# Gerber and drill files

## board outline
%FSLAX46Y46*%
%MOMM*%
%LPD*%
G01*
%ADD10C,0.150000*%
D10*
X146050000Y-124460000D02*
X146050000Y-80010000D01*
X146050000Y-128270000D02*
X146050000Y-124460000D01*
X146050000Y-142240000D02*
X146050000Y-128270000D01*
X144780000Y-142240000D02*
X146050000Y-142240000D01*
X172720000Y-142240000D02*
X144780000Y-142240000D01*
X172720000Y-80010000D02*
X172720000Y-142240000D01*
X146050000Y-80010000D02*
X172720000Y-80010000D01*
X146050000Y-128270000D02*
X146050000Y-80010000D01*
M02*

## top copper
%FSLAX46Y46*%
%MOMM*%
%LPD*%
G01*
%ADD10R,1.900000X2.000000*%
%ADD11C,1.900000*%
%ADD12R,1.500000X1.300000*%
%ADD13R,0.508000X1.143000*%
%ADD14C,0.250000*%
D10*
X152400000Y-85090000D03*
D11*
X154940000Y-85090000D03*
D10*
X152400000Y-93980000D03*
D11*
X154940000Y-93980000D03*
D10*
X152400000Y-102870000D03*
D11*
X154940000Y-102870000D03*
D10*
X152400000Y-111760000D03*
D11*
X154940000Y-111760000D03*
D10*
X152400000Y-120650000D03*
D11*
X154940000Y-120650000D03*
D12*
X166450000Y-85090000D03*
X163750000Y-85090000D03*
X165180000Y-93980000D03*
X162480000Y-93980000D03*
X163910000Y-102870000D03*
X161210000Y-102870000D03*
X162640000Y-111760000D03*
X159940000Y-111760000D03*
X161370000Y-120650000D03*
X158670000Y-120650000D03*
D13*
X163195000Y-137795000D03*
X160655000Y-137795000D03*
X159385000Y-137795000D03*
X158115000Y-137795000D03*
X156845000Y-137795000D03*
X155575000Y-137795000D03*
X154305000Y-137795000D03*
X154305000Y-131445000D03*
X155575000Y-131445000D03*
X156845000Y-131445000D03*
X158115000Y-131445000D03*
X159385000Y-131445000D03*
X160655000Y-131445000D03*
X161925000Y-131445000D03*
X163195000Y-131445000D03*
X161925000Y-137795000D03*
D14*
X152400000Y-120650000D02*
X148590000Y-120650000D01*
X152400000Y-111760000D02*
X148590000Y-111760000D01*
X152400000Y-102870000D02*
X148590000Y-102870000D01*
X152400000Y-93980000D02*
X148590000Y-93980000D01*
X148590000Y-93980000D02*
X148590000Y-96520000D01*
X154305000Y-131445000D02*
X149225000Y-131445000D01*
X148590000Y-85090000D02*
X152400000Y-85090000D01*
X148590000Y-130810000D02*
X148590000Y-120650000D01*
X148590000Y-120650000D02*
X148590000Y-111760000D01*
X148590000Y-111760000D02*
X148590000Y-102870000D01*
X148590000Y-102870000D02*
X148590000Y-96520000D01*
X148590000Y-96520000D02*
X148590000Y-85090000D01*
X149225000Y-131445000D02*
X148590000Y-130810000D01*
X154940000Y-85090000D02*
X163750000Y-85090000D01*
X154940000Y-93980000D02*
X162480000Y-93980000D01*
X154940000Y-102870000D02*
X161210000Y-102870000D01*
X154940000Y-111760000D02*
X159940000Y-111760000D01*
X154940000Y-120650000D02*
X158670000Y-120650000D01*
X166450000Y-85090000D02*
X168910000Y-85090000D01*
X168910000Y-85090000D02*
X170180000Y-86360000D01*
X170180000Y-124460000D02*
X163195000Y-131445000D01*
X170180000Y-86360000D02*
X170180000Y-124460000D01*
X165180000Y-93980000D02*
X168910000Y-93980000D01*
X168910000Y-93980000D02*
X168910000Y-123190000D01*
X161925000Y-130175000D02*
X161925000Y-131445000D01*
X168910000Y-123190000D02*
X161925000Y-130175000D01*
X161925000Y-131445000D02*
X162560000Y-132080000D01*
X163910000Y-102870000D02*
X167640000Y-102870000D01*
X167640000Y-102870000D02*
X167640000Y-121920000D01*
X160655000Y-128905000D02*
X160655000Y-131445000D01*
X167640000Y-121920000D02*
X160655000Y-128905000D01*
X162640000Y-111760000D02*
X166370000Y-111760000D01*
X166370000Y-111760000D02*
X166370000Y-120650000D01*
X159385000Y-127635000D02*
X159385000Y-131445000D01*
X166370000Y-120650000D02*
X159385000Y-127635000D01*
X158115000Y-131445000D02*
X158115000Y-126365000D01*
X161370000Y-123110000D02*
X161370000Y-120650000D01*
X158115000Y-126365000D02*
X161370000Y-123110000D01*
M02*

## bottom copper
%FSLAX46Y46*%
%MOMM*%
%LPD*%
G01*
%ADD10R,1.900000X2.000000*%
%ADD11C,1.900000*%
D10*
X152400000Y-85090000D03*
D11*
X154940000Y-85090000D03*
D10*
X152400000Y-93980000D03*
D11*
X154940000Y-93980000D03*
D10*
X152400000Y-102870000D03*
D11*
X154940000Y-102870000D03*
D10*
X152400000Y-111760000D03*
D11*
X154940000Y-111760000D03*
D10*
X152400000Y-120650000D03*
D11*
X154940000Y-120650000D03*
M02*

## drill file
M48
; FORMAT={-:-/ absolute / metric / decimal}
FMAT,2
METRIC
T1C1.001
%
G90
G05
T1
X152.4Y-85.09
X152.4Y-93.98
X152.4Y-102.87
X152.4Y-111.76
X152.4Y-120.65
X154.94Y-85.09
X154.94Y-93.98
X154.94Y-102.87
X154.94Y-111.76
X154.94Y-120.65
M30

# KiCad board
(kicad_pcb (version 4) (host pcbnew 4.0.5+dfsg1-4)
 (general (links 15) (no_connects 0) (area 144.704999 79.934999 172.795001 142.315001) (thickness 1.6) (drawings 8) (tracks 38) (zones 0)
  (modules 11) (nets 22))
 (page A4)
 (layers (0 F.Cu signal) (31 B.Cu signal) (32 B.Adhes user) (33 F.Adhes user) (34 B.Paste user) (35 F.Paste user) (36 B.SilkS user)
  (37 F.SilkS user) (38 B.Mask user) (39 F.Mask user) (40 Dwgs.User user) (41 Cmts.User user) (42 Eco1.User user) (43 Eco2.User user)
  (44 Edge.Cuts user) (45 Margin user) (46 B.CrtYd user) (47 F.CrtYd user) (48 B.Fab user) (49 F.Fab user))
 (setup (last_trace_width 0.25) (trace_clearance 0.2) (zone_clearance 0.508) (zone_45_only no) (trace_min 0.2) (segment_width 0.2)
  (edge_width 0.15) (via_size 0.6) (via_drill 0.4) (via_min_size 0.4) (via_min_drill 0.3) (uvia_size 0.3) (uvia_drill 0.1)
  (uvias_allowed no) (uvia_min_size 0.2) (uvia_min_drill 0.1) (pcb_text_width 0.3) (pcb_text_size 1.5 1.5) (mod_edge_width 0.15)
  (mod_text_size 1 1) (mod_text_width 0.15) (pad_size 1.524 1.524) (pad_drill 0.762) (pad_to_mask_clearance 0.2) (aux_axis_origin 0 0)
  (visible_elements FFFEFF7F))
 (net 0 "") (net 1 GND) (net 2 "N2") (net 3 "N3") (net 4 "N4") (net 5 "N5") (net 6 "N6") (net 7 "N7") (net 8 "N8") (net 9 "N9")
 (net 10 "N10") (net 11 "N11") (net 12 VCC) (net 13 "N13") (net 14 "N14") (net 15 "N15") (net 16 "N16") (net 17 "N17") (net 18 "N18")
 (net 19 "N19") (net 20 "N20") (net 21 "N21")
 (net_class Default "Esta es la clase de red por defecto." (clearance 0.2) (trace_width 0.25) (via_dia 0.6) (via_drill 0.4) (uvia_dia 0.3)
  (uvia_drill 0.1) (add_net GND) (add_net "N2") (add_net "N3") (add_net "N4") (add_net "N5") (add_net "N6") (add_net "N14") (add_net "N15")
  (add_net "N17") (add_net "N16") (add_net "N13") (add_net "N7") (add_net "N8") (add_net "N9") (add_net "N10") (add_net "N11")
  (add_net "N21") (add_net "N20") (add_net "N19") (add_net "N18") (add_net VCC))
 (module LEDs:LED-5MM (layer F.Cu) (at 152.4 85.09)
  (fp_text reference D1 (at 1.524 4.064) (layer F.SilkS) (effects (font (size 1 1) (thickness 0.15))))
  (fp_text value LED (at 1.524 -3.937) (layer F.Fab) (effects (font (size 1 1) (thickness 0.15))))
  (pad 1 thru_hole rect (at 0 0 90) (size 2 1.9) (drill 1.00076) (layers *.Cu *.Mask) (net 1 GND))
  (pad 2 thru_hole circle (at 2.54 0) (size 1.9 1.9) (drill 1.00076) (layers *.Cu *.Mask) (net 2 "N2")))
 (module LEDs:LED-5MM (layer F.Cu) (at 152.4 93.98)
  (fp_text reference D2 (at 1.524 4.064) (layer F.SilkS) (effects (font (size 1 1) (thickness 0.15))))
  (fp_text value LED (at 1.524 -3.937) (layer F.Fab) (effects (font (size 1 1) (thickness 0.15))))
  (pad 1 thru_hole rect (at 0 0 90) (size 2 1.9) (drill 1.00076) (layers *.Cu *.Mask) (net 1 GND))
  (pad 2 thru_hole circle (at 2.54 0) (size 1.9 1.9) (drill 1.00076) (layers *.Cu *.Mask) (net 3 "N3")))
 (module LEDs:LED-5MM (layer F.Cu) (at 152.4 102.87)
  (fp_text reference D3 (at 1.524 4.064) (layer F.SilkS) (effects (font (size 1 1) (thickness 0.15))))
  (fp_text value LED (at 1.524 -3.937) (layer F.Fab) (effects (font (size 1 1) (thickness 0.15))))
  (pad 1 thru_hole rect (at 0 0 90) (size 2 1.9) (drill 1.00076) (layers *.Cu *.Mask) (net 1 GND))
  (pad 2 thru_hole circle (at 2.54 0) (size 1.9 1.9) (drill 1.00076) (layers *.Cu *.Mask) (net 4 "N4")))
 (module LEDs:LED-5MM (layer F.Cu) (at 152.4 111.76)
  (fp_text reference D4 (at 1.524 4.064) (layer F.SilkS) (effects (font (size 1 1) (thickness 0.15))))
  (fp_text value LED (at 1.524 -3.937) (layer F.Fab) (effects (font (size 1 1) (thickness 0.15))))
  (pad 1 thru_hole rect (at 0 0 90) (size 2 1.9) (drill 1.00076) (layers *.Cu *.Mask) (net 1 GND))
  (pad 2 thru_hole circle (at 2.54 0) (size 1.9 1.9) (drill 1.00076) (layers *.Cu *.Mask) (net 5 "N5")))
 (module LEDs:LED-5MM (layer F.Cu) (at 152.4 120.65)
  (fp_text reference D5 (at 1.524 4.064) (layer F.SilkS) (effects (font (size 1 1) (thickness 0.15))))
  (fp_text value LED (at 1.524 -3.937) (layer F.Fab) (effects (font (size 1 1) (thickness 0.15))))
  (pad 1 thru_hole rect (at 0 0 90) (size 2 1.9) (drill 1.00076) (layers *.Cu *.Mask) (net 1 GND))
  (pad 2 thru_hole circle (at 2.54 0) (size 1.9 1.9) (drill 1.00076) (layers *.Cu *.Mask) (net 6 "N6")))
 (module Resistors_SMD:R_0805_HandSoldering (layer F.Cu) (at 165.1 85.09 180)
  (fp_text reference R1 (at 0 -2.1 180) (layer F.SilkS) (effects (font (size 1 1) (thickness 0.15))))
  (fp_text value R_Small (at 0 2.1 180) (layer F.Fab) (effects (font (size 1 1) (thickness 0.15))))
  (pad 1 smd rect (at -1.35 0 180) (size 1.5 1.3) (layers F.Cu F.Paste F.Mask) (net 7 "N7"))
  (pad 2 smd rect (at 1.35 0 180) (size 1.5 1.3) (layers F.Cu F.Paste F.Mask) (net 2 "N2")))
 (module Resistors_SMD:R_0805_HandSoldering (layer F.Cu) (at 163.83 93.98 180)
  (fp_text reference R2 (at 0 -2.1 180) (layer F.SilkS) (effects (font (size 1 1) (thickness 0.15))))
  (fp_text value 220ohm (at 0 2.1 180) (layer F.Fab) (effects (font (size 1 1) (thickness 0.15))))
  (pad 1 smd rect (at -1.35 0 180) (size 1.5 1.3) (layers F.Cu F.Paste F.Mask) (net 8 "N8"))
  (pad 2 smd rect (at 1.35 0 180) (size 1.5 1.3) (layers F.Cu F.Paste F.Mask) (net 3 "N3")))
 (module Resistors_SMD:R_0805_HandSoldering (layer F.Cu) (at 162.56 102.87 180)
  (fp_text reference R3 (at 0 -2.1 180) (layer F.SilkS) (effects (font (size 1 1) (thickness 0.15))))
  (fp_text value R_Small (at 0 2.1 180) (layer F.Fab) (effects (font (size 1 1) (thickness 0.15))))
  (pad 1 smd rect (at -1.35 0 180) (size 1.5 1.3) (layers F.Cu F.Paste F.Mask) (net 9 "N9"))
  (pad 2 smd rect (at 1.35 0 180) (size 1.5 1.3) (layers F.Cu F.Paste F.Mask) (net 4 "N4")))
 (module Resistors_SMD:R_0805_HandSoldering (layer F.Cu) (at 161.29 111.76 180)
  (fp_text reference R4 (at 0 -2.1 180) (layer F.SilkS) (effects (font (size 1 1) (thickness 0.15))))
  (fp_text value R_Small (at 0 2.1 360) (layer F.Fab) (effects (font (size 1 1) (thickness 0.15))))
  (pad 1 smd rect (at -1.35 0 180) (size 1.5 1.3) (layers F.Cu F.Paste F.Mask) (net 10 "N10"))
  (pad 2 smd rect (at 1.35 0 180) (size 1.5 1.3) (layers F.Cu F.Paste F.Mask) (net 5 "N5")))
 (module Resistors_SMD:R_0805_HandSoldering (layer F.Cu) (at 160.02 120.65 180)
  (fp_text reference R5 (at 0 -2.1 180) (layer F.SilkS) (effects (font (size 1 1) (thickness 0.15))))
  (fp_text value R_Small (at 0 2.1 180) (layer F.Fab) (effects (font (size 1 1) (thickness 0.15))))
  (pad 1 smd rect (at -1.35 0 180) (size 1.5 1.3) (layers F.Cu F.Paste F.Mask) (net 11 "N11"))
  (pad 2 smd rect (at 1.35 0 180) (size 1.5 1.3) (layers F.Cu F.Paste F.Mask) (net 6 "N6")))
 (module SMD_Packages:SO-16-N (layer F.Cu) (at 158.75 134.62 180)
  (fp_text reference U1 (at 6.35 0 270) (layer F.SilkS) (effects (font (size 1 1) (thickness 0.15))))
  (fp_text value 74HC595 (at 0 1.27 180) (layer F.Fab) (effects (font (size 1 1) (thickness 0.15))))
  (pad 16 smd rect (at -4.445 -3.175 180) (size 0.508 1.143) (layers F.Cu F.Paste F.Mask) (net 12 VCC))
  (pad 14 smd rect (at -1.905 -3.175 180) (size 0.508 1.143) (layers F.Cu F.Paste F.Mask) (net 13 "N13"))
  (pad 13 smd rect (at -0.635 -3.175 180) (size 0.508 1.143) (layers F.Cu F.Paste F.Mask) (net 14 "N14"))
  (pad 12 smd rect (at 0.635 -3.175 180) (size 0.508 1.143) (layers F.Cu F.Paste F.Mask) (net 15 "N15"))
  (pad 11 smd rect (at 1.905 -3.175 180) (size 0.508 1.143) (layers F.Cu F.Paste F.Mask) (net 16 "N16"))
  (pad 10 smd rect (at 3.175 -3.175 180) (size 0.508 1.143) (layers F.Cu F.Paste F.Mask) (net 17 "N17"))
  (pad 9 smd rect (at 4.445 -3.175 180) (size 0.508 1.143) (layers F.Cu F.Paste F.Mask) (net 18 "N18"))
  (pad 8 smd rect (at 4.445 3.175 180) (size 0.508 1.143) (layers F.Cu F.Paste F.Mask) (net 1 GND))
  (pad 7 smd rect (at 3.175 3.175 180) (size 0.508 1.143) (layers F.Cu F.Paste F.Mask) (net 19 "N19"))
  (pad 6 smd rect (at 1.905 3.175 180) (size 0.508 1.143) (layers F.Cu F.Paste F.Mask) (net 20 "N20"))
  (pad 5 smd rect (at 0.635 3.175 180) (size 0.508 1.143) (layers F.Cu F.Paste F.Mask) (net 11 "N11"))
  (pad 4 smd rect (at -0.635 3.175 180) (size 0.508 1.143) (layers F.Cu F.Paste F.Mask) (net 10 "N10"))
  (pad 3 smd rect (at -1.905 3.175 180) (size 0.508 1.143) (layers F.Cu F.Paste F.Mask) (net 9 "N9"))
  (pad 2 smd rect (at -3.175 3.175 180) (size 0.508 1.143) (layers F.Cu F.Paste F.Mask) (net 8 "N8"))
  (pad 1 smd rect (at -4.445 3.175 180) (size 0.508 1.143) (layers F.Cu F.Paste F.Mask) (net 7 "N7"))
  (pad 15 smd rect (at -3.175 -3.175 180) (size 0.508 1.143) (layers F.Cu F.Paste F.Mask) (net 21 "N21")))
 (gr_line (start 146.05 124.46) (end 146.05 80.01) (angle 90) (layer Edge.Cuts) (width 0.15))
 (gr_line (start 146.05 128.27) (end 146.05 124.46) (angle 90) (layer Edge.Cuts) (width 0.15))
 (gr_line (start 146.05 142.24) (end 146.05 128.27) (angle 90) (layer Edge.Cuts) (width 0.15))
 (gr_line (start 144.78 142.24) (end 146.05 142.24) (angle 90) (layer Edge.Cuts) (width 0.15))
 (gr_line (start 172.72 142.24) (end 144.78 142.24) (angle 90) (layer Edge.Cuts) (width 0.15))
 (gr_line (start 172.72 80.01) (end 172.72 142.24) (angle 90) (layer Edge.Cuts) (width 0.15))
 (gr_line (start 146.05 80.01) (end 172.72 80.01) (angle 90) (layer Edge.Cuts) (width 0.15))
 (gr_line (start 146.05 128.27) (end 146.05 80.01) (angle 90) (layer Edge.Cuts) (width 0.15))
 (segment (start 152.4 120.65) (end 148.59 120.65) (width 0.25) (layer F.Cu) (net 1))
 (segment (start 152.4 111.76) (end 148.59 111.76) (width 0.25) (layer F.Cu) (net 1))
 (segment (start 152.4 102.87) (end 148.59 102.87) (width 0.25) (layer F.Cu) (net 1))
 (segment (start 152.4 93.98) (end 148.59 93.98) (width 0.25) (layer F.Cu) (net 1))
 (segment (start 148.59 93.98) (end 148.59 96.52) (width 0.25) (layer F.Cu) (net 1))
 (segment (start 154.305 131.445) (end 149.225 131.445) (width 0.25) (layer F.Cu) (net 1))
 (segment (start 148.59 85.09) (end 152.4 85.09) (width 0.25) (layer F.Cu) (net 1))
 (segment (start 148.59 130.81) (end 148.59 120.65) (width 0.25) (layer F.Cu) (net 1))
 (segment (start 148.59 120.65) (end 148.59 111.76) (width 0.25) (layer F.Cu) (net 1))
 (segment (start 148.59 111.76) (end 148.59 102.87) (width 0.25) (layer F.Cu) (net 1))
 (segment (start 148.59 102.87) (end 148.59 96.52) (width 0.25) (layer F.Cu) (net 1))
 (segment (start 148.59 96.52) (end 148.59 85.09) (width 0.25) (layer F.Cu) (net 1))
 (segment (start 149.225 131.445) (end 148.59 130.81) (width 0.25) (layer F.Cu) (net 1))
 (segment (start 154.94 85.09) (end 163.75 85.09) (width 0.25) (layer F.Cu) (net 2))
 (segment (start 154.94 93.98) (end 162.48 93.98) (width 0.25) (layer F.Cu) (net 3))
 (segment (start 154.94 102.87) (end 161.21 102.87) (width 0.25) (layer F.Cu) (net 4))
 (segment (start 154.94 111.76) (end 159.94 111.76) (width 0.25) (layer F.Cu) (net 5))
 (segment (start 154.94 120.65) (end 158.67 120.65) (width 0.25) (layer F.Cu) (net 6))
 (segment (start 166.45 85.09) (end 168.91 85.09) (width 0.25) (layer F.Cu) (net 7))
 (segment (start 168.91 85.09) (end 170.18 86.36) (width 0.25) (layer F.Cu) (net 7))
 (segment (start 170.18 124.46) (end 163.195 131.445) (width 0.25) (layer F.Cu) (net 7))
 (segment (start 170.18 86.36) (end 170.18 124.46) (width 0.25) (layer F.Cu) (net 7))
 (segment (start 165.18 93.98) (end 168.91 93.98) (width 0.25) (layer F.Cu) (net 8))
 (segment (start 168.91 93.98) (end 168.91 123.19) (width 0.25) (layer F.Cu) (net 8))
 (segment (start 161.925 130.175) (end 161.925 131.445) (width 0.25) (layer F.Cu) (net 8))
 (segment (start 168.91 123.19) (end 161.925 130.175) (width 0.25) (layer F.Cu) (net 8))
 (segment (start 161.925 131.445) (end 162.56 132.08) (width 0.25) (layer F.Cu) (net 8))
 (segment (start 163.91 102.87) (end 167.64 102.87) (width 0.25) (layer F.Cu) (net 9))
 (segment (start 167.64 102.87) (end 167.64 121.92) (width 0.25) (layer F.Cu) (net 9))
 (segment (start 160.655 128.905) (end 160.655 131.445) (width 0.25) (layer F.Cu) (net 9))
 (segment (start 167.64 121.92) (end 160.655 128.905) (width 0.25) (layer F.Cu) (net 9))
 (segment (start 162.64 111.76) (end 166.37 111.76) (width 0.25) (layer F.Cu) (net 10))
 (segment (start 166.37 111.76) (end 166.37 120.65) (width 0.25) (layer F.Cu) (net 10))
 (segment (start 159.385 127.635) (end 159.385 131.445) (width 0.25) (layer F.Cu) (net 10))
 (segment (start 166.37 120.65) (end 159.385 127.635) (width 0.25) (layer F.Cu) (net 10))
 (segment (start 158.115 131.445) (end 158.115 126.365) (width 0.25) (layer F.Cu) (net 11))
 (segment (start 161.37 123.11) (end 161.37 120.65) (width 0.25) (layer F.Cu) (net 11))
 (segment (start 158.115 126.365) (end 161.37 123.11) (width 0.25) (layer F.Cu) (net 11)))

